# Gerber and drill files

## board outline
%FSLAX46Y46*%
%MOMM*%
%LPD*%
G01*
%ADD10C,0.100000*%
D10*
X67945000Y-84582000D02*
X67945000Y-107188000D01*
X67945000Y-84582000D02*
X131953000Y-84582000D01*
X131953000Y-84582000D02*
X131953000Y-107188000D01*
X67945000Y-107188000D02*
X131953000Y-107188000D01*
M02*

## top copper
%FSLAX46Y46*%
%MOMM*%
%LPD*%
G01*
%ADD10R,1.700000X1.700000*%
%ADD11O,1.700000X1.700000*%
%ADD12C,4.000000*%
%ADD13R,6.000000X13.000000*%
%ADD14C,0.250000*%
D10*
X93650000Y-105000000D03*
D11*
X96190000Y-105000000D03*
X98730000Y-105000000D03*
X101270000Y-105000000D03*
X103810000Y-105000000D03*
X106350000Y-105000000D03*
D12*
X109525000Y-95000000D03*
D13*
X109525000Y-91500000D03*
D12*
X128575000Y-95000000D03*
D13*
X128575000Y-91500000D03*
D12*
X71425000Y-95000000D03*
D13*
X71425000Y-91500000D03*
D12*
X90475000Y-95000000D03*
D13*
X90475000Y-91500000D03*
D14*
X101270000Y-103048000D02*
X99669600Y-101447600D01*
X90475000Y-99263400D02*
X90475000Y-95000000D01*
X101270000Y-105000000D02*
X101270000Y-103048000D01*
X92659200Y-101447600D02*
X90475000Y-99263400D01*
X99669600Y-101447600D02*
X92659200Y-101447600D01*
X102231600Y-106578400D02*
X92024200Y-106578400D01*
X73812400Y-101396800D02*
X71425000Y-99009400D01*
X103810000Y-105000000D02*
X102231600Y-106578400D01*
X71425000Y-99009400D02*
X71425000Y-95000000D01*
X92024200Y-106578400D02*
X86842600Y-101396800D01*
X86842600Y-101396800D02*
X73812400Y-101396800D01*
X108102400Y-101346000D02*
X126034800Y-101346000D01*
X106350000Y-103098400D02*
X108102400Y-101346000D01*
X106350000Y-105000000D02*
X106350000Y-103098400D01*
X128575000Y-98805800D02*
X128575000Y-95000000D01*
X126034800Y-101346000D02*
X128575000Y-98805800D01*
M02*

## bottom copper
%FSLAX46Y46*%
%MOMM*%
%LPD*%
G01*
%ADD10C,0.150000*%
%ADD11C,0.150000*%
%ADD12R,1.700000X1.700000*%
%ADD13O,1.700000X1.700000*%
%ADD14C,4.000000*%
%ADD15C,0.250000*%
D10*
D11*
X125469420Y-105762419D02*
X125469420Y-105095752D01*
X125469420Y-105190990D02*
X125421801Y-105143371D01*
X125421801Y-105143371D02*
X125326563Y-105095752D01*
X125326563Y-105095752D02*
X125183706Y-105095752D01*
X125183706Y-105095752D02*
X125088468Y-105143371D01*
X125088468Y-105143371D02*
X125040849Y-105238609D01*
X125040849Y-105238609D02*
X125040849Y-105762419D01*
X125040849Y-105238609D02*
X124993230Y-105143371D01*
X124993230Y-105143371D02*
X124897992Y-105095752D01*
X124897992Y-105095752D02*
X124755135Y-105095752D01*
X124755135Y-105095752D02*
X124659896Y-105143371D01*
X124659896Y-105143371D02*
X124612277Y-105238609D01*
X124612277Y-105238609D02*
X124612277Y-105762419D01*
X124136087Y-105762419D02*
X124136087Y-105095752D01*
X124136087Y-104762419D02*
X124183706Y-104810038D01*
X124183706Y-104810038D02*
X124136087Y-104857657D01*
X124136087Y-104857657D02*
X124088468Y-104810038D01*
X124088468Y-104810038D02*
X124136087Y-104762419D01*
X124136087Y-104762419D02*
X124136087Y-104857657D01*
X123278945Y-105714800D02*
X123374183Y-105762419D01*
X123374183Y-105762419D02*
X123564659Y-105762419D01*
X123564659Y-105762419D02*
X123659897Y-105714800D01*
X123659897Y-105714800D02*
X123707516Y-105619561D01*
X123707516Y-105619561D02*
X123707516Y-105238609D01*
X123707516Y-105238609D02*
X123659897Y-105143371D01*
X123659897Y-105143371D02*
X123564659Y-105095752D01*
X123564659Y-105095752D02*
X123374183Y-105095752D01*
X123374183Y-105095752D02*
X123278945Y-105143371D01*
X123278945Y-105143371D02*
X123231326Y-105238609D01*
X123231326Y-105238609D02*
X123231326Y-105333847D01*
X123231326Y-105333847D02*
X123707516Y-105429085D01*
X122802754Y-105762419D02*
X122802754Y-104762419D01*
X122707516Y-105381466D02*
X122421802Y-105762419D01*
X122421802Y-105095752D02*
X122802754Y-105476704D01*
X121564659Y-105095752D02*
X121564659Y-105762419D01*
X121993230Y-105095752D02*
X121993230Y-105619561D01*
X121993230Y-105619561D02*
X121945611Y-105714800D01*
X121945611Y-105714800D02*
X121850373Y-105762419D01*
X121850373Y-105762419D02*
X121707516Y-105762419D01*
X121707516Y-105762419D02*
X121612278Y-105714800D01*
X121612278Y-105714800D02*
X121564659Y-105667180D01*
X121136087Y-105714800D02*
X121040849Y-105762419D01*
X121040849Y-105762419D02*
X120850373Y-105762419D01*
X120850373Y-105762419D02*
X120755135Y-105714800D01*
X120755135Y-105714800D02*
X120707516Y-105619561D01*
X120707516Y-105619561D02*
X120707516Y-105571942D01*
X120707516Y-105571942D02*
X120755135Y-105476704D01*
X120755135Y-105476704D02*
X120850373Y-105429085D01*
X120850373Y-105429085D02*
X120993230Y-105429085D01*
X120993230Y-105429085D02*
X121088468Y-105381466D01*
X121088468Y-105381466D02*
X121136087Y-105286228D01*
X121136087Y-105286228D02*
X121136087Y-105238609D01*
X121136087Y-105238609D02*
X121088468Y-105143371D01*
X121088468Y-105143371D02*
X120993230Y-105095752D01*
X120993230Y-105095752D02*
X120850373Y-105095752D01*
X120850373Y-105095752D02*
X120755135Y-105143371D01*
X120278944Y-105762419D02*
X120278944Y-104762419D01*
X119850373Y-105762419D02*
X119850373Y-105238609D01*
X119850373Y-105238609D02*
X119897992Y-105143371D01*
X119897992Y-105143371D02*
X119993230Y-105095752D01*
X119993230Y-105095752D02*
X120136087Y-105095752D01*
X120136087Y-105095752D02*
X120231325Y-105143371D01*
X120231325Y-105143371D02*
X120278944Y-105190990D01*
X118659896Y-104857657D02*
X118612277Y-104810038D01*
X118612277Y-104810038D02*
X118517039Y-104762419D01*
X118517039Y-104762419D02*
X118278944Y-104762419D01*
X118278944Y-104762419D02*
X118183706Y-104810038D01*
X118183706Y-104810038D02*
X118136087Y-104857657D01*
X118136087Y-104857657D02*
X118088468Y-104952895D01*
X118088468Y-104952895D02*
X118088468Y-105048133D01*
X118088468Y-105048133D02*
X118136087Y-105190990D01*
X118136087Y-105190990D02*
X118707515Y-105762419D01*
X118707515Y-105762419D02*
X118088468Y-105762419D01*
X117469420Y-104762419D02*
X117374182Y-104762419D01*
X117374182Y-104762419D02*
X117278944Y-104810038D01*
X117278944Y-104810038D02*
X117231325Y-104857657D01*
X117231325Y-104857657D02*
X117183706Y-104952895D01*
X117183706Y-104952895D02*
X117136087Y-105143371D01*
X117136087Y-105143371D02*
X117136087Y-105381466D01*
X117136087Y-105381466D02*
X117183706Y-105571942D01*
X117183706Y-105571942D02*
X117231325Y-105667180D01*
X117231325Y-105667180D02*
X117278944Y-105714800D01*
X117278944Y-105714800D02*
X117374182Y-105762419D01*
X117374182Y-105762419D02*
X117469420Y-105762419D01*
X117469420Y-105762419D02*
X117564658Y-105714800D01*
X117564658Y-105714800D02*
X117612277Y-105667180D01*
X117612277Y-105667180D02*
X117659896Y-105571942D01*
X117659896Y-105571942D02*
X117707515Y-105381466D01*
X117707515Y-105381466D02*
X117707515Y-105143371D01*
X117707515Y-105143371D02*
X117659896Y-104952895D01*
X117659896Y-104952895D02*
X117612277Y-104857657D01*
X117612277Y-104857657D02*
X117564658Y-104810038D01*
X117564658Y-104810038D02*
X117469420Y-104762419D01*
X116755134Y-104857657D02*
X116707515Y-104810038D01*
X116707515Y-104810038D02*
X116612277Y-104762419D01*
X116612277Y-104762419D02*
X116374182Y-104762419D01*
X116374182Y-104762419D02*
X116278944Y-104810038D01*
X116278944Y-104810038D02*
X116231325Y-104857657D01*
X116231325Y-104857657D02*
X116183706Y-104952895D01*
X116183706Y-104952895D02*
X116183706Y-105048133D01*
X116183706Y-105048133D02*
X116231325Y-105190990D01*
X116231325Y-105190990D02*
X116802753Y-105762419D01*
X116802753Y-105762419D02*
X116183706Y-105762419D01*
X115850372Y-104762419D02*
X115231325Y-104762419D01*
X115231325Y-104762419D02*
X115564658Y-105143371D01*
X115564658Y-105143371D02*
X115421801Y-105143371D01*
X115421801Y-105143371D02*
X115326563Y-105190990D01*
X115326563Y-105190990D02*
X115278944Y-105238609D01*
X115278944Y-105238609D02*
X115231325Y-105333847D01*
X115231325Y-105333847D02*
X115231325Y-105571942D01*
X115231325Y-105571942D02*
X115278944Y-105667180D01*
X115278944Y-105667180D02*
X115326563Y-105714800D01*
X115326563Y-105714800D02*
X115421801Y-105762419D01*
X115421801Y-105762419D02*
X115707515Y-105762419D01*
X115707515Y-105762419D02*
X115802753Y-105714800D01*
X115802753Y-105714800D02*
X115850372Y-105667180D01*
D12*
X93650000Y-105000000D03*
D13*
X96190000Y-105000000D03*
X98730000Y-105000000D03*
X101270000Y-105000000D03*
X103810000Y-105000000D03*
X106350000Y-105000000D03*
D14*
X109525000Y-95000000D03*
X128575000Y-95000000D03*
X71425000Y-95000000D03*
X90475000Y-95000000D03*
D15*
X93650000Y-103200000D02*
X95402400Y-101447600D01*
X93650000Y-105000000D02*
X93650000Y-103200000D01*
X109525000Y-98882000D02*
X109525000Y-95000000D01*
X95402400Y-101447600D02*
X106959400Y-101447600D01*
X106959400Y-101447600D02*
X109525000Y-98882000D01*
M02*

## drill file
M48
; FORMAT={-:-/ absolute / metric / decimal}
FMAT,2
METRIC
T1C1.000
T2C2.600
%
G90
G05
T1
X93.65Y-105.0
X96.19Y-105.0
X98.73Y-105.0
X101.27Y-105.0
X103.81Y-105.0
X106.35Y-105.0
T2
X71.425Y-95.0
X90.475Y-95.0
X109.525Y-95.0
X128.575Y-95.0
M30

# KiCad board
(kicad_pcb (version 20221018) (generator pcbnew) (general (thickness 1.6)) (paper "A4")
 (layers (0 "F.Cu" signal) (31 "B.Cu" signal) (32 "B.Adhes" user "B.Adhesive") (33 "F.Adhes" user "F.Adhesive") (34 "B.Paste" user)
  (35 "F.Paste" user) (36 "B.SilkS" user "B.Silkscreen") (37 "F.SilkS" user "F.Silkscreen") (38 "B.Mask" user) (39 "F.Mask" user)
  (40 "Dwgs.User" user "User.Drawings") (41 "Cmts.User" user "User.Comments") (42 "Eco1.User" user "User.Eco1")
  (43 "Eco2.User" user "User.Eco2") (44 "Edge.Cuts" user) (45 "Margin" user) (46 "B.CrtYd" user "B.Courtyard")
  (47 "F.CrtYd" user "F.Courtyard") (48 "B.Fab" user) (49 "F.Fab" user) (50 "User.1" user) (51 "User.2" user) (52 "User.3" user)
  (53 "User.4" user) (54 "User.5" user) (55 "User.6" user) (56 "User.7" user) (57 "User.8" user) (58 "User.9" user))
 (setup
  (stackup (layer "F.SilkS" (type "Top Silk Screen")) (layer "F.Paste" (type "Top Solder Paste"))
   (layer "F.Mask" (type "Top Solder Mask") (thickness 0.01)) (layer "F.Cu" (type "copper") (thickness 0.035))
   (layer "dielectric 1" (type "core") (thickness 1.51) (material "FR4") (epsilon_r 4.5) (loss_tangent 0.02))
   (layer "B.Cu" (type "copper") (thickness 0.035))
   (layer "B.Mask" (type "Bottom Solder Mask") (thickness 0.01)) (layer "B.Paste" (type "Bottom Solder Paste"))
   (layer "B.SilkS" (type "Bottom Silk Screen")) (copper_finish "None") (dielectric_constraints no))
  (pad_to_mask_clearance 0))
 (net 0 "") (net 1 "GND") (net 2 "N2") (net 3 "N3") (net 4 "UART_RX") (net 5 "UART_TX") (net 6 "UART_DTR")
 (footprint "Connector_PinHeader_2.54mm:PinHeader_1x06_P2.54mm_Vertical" (layer "F.Cu") (at 93.65 105 90)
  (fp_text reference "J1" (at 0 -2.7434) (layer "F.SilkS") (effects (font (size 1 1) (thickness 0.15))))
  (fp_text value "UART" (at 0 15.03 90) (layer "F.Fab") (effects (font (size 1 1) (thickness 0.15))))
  (pad "1" thru_hole rect (at 0 0 90) (size 1.7 1.7) (drill 1) (layers "*.Cu" "*.Mask") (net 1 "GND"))
  (pad "2" thru_hole oval (at 0 2.54 90) (size 1.7 1.7) (drill 1) (layers "*.Cu" "*.Mask") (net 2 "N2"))
  (pad "3" thru_hole oval (at 0 5.08 90) (size 1.7 1.7) (drill 1) (layers "*.Cu" "*.Mask") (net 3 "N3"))
  (pad "4" thru_hole oval (at 0 7.62 90) (size 1.7 1.7) (drill 1) (layers "*.Cu" "*.Mask") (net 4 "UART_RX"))
  (pad "5" thru_hole oval (at 0 10.16 90) (size 1.7 1.7) (drill 1) (layers "*.Cu" "*.Mask") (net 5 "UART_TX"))
  (pad "6" thru_hole oval (at 0 12.7 90) (size 1.7 1.7) (drill 1) (layers "*.Cu" "*.Mask") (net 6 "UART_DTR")))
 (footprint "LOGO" (layer "F.Cu") (at 113.411 104.013)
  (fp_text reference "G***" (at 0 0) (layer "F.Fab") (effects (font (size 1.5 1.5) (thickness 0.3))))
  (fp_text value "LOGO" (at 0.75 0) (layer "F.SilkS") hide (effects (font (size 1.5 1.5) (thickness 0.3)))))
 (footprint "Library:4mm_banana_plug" (layer "F.Cu") (at 109.525 95 180)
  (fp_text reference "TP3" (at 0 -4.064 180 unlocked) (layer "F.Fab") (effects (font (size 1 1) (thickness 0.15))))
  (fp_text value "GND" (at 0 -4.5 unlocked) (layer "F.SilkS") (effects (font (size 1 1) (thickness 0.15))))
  (pad "1" thru_hole circle (at 0 0 180) (size 4 4) (drill 2.6) (layers "*.Cu" "*.Mask") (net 1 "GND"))
  (pad "1" smd rect (at 0 0 180) (size 6 13) (drill (offset 0 3.5)) (layers "F.Cu" "F.Mask") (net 1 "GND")))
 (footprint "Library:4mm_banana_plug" (layer "F.Cu") (at 128.575 95 180)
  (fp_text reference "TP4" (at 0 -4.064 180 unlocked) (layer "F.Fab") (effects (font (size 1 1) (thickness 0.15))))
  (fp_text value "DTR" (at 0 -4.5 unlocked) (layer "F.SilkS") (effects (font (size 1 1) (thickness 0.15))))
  (pad "1" thru_hole circle (at 0 0 180) (size 4 4) (drill 2.6) (layers "*.Cu" "*.Mask") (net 6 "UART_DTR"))
  (pad "1" smd rect (at 0 0 180) (size 6 13) (drill (offset 0 3.5)) (layers "F.Cu" "F.Mask") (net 6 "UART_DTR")))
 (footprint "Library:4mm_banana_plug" (layer "F.Cu") (at 71.425 95 180)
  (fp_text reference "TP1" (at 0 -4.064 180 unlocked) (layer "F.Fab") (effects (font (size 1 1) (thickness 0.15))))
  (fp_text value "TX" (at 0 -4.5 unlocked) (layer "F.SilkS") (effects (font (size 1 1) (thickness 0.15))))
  (pad "1" thru_hole circle (at 0 0 180) (size 4 4) (drill 2.6) (layers "*.Cu" "*.Mask") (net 5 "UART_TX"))
  (pad "1" smd rect (at 0 0 180) (size 6 13) (drill (offset 0 3.5)) (layers "F.Cu" "F.Mask") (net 5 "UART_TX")))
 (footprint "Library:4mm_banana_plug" (layer "F.Cu") (at 90.475 95 180)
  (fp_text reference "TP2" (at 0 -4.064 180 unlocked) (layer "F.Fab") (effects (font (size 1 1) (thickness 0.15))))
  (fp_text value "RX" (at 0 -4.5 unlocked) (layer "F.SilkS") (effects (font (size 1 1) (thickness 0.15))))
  (pad "1" thru_hole circle (at 0 0 180) (size 4 4) (drill 2.6) (layers "*.Cu" "*.Mask") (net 4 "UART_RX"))
  (pad "1" smd rect (at 0 0 180) (size 6 13) (drill (offset 0 3.5)) (layers "F.Cu" "F.Mask") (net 4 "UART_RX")))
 (gr_line (start 67.945 84.582) (end 67.945 107.188) (stroke (width 0.1) (type default)) (layer "Edge.Cuts"))
 (gr_line (start 67.945 84.582) (end 131.953 84.582) (stroke (width 0.1) (type default)) (layer "Edge.Cuts"))
 (gr_line (start 131.953 84.582) (end 131.953 107.188) (stroke (width 0.1) (type default)) (layer "Edge.Cuts"))
 (gr_line (start 67.945 107.188) (end 131.953 107.188) (stroke (width 0.1) (type default)) (layer "Edge.Cuts"))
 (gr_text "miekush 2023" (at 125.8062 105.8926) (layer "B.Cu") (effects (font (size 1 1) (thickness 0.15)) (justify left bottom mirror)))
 (segment (start 93.65 103.2) (end 95.4024 101.4476) (width 0.25) (layer "B.Cu") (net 1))
 (segment (start 93.65 105) (end 93.65 103.2) (width 0.25) (layer "B.Cu") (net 1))
 (segment (start 109.525 98.882) (end 109.525 95) (width 0.25) (layer "B.Cu") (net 1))
 (segment (start 95.4024 101.4476) (end 106.9594 101.4476) (width 0.25) (layer "B.Cu") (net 1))
 (segment (start 106.9594 101.4476) (end 109.525 98.882) (width 0.25) (layer "B.Cu") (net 1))
 (segment (start 101.27 103.048) (end 99.6696 101.4476) (width 0.25) (layer "F.Cu") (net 4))
 (segment (start 90.475 99.2634) (end 90.475 95) (width 0.25) (layer "F.Cu") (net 4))
 (segment (start 101.27 105) (end 101.27 103.048) (width 0.25) (layer "F.Cu") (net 4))
 (segment (start 92.6592 101.4476) (end 90.475 99.2634) (width 0.25) (layer "F.Cu") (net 4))
 (segment (start 99.6696 101.4476) (end 92.6592 101.4476) (width 0.25) (layer "F.Cu") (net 4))
 (segment (start 102.2316 106.5784) (end 92.0242 106.5784) (width 0.25) (layer "F.Cu") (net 5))
 (segment (start 73.8124 101.3968) (end 71.425 99.0094) (width 0.25) (layer "F.Cu") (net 5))
 (segment (start 103.81 105) (end 102.2316 106.5784) (width 0.25) (layer "F.Cu") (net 5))
 (segment (start 71.425 99.0094) (end 71.425 95) (width 0.25) (layer "F.Cu") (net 5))
 (segment (start 92.0242 106.5784) (end 86.8426 101.3968) (width 0.25) (layer "F.Cu") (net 5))
 (segment (start 86.8426 101.3968) (end 73.8124 101.3968) (width 0.25) (layer "F.Cu") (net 5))
 (segment (start 108.1024 101.346) (end 126.0348 101.346) (width 0.25) (layer "F.Cu") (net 6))
 (segment (start 106.35 103.0984) (end 108.1024 101.346) (width 0.25) (layer "F.Cu") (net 6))
 (segment (start 106.35 105) (end 106.35 103.0984) (width 0.25) (layer "F.Cu") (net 6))
 (segment (start 128.575 98.8058) (end 128.575 95) (width 0.25) (layer "F.Cu") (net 6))
 (segment (start 126.0348 101.346) (end 128.575 98.8058) (width 0.25) (layer "F.Cu") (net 6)))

